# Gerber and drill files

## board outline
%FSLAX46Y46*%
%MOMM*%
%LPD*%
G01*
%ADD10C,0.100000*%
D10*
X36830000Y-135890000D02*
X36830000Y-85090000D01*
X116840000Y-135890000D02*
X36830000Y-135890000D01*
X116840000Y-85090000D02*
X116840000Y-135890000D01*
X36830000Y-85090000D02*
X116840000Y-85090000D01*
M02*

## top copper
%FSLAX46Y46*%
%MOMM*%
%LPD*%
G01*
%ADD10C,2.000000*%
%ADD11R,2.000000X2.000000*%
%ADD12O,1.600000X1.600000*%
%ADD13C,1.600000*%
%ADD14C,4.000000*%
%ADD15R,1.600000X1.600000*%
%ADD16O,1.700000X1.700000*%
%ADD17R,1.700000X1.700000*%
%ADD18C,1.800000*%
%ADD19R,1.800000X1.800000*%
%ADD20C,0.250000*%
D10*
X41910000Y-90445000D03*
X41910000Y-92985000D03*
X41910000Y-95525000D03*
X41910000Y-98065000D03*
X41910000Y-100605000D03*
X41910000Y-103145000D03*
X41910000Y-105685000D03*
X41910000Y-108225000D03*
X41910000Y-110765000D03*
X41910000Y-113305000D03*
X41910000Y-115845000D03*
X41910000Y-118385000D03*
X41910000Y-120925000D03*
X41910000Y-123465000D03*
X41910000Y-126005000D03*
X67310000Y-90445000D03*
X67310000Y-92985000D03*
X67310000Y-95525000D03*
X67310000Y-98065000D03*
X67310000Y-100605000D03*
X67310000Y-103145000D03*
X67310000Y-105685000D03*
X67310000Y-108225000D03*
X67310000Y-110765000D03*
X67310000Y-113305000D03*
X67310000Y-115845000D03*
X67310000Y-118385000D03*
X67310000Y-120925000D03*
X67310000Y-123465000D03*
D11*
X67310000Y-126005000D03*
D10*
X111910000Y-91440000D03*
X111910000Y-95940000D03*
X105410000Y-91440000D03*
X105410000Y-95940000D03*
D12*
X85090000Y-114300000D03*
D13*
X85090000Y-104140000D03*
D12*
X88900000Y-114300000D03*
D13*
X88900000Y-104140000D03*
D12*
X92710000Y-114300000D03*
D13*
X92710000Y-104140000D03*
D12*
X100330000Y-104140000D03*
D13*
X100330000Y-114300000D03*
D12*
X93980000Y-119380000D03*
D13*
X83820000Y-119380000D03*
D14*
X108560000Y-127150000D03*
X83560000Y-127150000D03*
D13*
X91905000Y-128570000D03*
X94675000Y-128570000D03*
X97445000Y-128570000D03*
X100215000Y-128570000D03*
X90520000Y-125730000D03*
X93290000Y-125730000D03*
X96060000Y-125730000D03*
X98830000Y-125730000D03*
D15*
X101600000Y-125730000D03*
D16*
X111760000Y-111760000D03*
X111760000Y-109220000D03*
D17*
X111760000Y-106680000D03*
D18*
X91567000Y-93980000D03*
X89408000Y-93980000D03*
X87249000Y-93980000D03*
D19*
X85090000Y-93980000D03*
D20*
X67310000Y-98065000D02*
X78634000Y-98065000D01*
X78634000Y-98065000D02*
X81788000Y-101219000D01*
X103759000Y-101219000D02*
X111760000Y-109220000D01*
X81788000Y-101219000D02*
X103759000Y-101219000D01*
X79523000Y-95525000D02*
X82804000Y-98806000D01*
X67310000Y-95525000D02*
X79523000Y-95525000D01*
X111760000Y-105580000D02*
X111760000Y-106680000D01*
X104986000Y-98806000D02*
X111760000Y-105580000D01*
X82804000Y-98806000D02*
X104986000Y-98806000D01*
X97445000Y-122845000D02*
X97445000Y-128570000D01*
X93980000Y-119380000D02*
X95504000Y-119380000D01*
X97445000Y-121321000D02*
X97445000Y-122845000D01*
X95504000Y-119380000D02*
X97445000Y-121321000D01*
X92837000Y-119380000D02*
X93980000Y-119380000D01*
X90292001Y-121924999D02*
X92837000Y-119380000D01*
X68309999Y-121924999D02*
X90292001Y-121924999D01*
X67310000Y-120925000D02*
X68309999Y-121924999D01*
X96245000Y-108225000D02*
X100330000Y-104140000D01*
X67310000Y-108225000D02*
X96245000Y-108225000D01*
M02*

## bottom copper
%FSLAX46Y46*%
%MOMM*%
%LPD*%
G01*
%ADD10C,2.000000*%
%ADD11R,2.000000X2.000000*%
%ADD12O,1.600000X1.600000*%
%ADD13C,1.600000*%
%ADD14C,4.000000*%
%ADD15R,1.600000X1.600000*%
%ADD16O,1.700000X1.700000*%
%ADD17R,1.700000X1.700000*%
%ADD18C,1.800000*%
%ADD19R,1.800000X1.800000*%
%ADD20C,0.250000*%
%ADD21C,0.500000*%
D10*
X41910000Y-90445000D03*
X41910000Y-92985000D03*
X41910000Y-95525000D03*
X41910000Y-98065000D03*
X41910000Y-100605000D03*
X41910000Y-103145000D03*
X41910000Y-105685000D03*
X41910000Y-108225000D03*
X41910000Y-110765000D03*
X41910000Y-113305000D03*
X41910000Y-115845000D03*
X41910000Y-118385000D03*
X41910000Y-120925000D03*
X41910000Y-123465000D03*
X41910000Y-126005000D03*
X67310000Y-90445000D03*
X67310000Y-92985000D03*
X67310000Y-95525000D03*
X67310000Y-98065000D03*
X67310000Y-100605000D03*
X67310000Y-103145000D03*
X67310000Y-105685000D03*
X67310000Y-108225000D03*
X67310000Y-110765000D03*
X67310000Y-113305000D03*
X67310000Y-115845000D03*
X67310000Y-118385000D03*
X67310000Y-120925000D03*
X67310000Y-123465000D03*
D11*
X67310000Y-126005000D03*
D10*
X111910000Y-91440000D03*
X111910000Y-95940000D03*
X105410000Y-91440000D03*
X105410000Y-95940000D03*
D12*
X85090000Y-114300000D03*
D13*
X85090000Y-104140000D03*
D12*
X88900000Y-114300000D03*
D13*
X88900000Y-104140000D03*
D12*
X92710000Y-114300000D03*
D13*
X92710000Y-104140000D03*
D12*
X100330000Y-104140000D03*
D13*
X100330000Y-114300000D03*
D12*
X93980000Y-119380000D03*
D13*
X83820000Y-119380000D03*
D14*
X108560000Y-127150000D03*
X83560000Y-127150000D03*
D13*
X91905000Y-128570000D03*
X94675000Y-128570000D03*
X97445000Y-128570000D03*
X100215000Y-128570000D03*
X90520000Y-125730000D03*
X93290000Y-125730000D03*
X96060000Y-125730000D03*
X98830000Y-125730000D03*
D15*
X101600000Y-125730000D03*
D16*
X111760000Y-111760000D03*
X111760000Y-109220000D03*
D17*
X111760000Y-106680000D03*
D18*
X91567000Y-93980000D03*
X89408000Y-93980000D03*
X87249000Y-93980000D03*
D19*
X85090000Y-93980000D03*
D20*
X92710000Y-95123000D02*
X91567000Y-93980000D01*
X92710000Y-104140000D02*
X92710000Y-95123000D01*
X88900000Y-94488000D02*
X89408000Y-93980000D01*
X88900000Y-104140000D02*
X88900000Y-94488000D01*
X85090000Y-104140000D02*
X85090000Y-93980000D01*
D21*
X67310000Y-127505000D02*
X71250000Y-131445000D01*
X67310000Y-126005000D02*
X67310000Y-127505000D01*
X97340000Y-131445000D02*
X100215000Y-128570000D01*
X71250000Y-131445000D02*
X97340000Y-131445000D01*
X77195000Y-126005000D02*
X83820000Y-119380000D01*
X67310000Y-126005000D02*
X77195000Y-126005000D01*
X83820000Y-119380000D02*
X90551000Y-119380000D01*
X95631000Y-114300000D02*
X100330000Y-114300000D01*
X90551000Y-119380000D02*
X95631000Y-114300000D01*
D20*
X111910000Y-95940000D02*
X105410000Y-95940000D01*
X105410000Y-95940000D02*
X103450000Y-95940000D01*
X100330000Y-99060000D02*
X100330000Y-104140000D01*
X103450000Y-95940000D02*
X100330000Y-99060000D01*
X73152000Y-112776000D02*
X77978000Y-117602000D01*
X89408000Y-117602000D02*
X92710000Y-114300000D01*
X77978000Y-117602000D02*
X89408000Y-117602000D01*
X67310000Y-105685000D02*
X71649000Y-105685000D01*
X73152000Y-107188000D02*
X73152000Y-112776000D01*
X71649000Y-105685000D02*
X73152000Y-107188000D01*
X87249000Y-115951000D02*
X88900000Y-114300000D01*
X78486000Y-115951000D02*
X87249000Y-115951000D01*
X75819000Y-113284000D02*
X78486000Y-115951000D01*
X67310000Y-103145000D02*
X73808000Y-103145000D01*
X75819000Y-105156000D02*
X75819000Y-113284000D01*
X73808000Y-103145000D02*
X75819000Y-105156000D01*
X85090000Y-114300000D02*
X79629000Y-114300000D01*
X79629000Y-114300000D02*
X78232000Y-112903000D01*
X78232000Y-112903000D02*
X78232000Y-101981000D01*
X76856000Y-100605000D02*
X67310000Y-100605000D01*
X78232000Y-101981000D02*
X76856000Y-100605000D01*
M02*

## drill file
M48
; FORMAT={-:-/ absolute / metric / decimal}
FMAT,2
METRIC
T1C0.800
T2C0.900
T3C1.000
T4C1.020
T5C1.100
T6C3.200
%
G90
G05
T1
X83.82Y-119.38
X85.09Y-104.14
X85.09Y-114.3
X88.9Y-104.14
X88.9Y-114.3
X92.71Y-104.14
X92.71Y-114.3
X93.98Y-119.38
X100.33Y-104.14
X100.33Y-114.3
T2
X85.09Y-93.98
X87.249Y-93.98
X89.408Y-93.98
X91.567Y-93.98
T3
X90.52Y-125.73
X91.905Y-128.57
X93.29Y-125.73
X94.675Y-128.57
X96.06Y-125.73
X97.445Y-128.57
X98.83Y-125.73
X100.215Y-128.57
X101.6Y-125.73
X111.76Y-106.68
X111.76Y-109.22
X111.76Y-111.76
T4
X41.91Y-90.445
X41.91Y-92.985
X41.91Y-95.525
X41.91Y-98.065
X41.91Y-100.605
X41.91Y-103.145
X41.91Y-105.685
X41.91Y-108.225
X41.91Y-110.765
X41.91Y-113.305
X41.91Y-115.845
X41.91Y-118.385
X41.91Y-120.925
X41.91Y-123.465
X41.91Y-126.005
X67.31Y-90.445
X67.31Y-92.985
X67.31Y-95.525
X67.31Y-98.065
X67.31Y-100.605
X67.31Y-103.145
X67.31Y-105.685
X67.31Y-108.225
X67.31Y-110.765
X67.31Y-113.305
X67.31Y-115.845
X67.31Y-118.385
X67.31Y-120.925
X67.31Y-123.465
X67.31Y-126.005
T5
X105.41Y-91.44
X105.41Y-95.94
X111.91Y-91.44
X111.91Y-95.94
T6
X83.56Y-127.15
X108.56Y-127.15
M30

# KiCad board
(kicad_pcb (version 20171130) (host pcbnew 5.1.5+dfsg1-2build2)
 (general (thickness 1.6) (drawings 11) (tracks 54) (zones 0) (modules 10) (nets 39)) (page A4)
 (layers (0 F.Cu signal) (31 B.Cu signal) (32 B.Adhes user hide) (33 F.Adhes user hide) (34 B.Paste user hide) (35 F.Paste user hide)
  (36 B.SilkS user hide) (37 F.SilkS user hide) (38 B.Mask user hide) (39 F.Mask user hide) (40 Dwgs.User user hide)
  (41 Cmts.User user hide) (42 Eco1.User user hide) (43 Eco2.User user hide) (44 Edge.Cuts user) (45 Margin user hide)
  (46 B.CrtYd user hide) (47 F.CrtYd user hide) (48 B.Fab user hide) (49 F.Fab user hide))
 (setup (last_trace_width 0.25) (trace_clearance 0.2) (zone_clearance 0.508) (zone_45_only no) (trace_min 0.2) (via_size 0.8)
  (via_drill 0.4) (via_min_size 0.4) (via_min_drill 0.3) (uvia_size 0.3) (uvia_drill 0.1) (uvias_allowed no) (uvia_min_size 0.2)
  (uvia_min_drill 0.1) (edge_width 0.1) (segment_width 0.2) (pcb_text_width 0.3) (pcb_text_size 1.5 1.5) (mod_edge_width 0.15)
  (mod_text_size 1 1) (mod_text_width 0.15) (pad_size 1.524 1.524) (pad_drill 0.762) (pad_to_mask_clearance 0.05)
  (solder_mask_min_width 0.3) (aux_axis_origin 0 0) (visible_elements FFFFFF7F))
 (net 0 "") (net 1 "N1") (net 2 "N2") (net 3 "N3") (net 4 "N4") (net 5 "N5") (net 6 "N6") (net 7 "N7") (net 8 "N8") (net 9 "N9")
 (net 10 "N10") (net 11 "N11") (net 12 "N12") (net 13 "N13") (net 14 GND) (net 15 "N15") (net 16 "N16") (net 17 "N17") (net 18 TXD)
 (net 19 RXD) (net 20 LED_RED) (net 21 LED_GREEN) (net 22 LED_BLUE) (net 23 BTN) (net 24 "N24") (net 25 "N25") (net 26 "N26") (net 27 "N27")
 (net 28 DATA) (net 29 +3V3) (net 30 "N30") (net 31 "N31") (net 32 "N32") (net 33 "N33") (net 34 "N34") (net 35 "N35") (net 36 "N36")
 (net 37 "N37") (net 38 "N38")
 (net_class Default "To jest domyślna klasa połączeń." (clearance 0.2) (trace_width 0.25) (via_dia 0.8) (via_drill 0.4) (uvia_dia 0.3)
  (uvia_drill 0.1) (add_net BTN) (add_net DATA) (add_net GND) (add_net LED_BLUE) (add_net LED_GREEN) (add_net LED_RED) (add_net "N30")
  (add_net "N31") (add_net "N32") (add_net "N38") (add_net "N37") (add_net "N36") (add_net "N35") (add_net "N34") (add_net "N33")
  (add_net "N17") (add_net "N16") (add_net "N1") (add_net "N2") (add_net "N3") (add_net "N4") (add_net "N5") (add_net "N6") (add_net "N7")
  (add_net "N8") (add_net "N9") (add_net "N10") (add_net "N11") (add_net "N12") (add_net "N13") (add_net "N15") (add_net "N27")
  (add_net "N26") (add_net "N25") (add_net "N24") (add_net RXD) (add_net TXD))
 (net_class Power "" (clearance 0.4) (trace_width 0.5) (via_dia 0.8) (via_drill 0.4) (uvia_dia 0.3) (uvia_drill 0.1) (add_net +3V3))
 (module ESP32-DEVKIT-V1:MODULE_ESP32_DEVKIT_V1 (layer F.Cu) (at 54.61 110.49 180)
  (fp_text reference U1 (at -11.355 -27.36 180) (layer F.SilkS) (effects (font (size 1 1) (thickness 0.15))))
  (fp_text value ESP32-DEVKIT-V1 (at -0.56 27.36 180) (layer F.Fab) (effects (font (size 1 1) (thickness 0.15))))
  (pad 16 thru_hole circle (at 12.7 20.045 180) (size 2 2) (drill 1.02) (layers *.Cu *.Mask) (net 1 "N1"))
  (pad 17 thru_hole circle (at 12.7 17.505 180) (size 2 2) (drill 1.02) (layers *.Cu *.Mask) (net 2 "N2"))
  (pad 18 thru_hole circle (at 12.7 14.965 180) (size 2 2) (drill 1.02) (layers *.Cu *.Mask) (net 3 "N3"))
  (pad 19 thru_hole circle (at 12.7 12.425 180) (size 2 2) (drill 1.02) (layers *.Cu *.Mask) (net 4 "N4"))
  (pad 20 thru_hole circle (at 12.7 9.885 180) (size 2 2) (drill 1.02) (layers *.Cu *.Mask) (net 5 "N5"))
  (pad 21 thru_hole circle (at 12.7 7.345 180) (size 2 2) (drill 1.02) (layers *.Cu *.Mask) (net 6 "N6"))
  (pad 22 thru_hole circle (at 12.7 4.805 180) (size 2 2) (drill 1.02) (layers *.Cu *.Mask) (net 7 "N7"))
  (pad 23 thru_hole circle (at 12.7 2.265 180) (size 2 2) (drill 1.02) (layers *.Cu *.Mask) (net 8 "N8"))
  (pad 24 thru_hole circle (at 12.7 -0.275 180) (size 2 2) (drill 1.02) (layers *.Cu *.Mask) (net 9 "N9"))
  (pad 25 thru_hole circle (at 12.7 -2.815 180) (size 2 2) (drill 1.02) (layers *.Cu *.Mask) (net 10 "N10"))
  (pad 26 thru_hole circle (at 12.7 -5.355 180) (size 2 2) (drill 1.02) (layers *.Cu *.Mask) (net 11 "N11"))
  (pad 27 thru_hole circle (at 12.7 -7.895 180) (size 2 2) (drill 1.02) (layers *.Cu *.Mask) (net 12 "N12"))
  (pad 28 thru_hole circle (at 12.7 -10.435 180) (size 2 2) (drill 1.02) (layers *.Cu *.Mask) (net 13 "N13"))
  (pad 29 thru_hole circle (at 12.7 -12.975 180) (size 2 2) (drill 1.02) (layers *.Cu *.Mask) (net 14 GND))
  (pad 30 thru_hole circle (at 12.7 -15.515 180) (size 2 2) (drill 1.02) (layers *.Cu *.Mask) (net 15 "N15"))
  (pad 15 thru_hole circle (at -12.7 20.045 180) (size 2 2) (drill 1.02) (layers *.Cu *.Mask) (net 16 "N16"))
  (pad 14 thru_hole circle (at -12.7 17.505 180) (size 2 2) (drill 1.02) (layers *.Cu *.Mask) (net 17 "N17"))
  (pad 13 thru_hole circle (at -12.7 14.965 180) (size 2 2) (drill 1.02) (layers *.Cu *.Mask) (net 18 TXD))
  (pad 12 thru_hole circle (at -12.7 12.425 180) (size 2 2) (drill 1.02) (layers *.Cu *.Mask) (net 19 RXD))
  (pad 11 thru_hole circle (at -12.7 9.885 180) (size 2 2) (drill 1.02) (layers *.Cu *.Mask) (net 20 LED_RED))
  (pad 10 thru_hole circle (at -12.7 7.345 180) (size 2 2) (drill 1.02) (layers *.Cu *.Mask) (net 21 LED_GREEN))
  (pad 9 thru_hole circle (at -12.7 4.805 180) (size 2 2) (drill 1.02) (layers *.Cu *.Mask) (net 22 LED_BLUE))
  (pad 8 thru_hole circle (at -12.7 2.265 180) (size 2 2) (drill 1.02) (layers *.Cu *.Mask) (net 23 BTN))
  (pad 7 thru_hole circle (at -12.7 -0.275 180) (size 2 2) (drill 1.02) (layers *.Cu *.Mask) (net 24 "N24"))
  (pad 6 thru_hole circle (at -12.7 -2.815 180) (size 2 2) (drill 1.02) (layers *.Cu *.Mask) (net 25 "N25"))
  (pad 5 thru_hole circle (at -12.7 -5.355 180) (size 2 2) (drill 1.02) (layers *.Cu *.Mask) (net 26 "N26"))
  (pad 4 thru_hole circle (at -12.7 -7.895 180) (size 2 2) (drill 1.02) (layers *.Cu *.Mask) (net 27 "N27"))
  (pad 3 thru_hole circle (at -12.7 -10.435 180) (size 2 2) (drill 1.02) (layers *.Cu *.Mask) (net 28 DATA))
  (pad 2 thru_hole circle (at -12.7 -12.975 180) (size 2 2) (drill 1.02) (layers *.Cu *.Mask) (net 14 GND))
  (pad 1 thru_hole rect (at -12.7 -15.515 180) (size 2 2) (drill 1.02) (layers *.Cu *.Mask) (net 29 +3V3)))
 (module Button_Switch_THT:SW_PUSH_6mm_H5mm (layer F.Cu) (at 105.41 91.44)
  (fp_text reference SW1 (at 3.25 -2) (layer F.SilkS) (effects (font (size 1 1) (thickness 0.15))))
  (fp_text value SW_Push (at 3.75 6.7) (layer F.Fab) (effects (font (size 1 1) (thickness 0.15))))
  (pad 1 thru_hole circle (at 6.5 0 90) (size 2 2) (drill 1.1) (layers *.Cu *.Mask) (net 14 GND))
  (pad 2 thru_hole circle (at 6.5 4.5 90) (size 2 2) (drill 1.1) (layers *.Cu *.Mask) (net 23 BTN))
  (pad 1 thru_hole circle (at 0 0 90) (size 2 2) (drill 1.1) (layers *.Cu *.Mask) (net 14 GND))
  (pad 2 thru_hole circle (at 0 4.5 90) (size 2 2) (drill 1.1) (layers *.Cu *.Mask) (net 23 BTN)))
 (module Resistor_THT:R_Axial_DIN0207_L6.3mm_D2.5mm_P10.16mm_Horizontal (layer F.Cu) (at 85.09 104.14 270)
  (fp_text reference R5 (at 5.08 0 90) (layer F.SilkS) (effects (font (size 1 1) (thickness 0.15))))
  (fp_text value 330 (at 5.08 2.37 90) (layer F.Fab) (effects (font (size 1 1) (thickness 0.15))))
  (pad 2 thru_hole oval (at 10.16 0 270) (size 1.6 1.6) (drill 0.8) (layers *.Cu *.Mask) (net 20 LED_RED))
  (pad 1 thru_hole circle (at 0 0 270) (size 1.6 1.6) (drill 0.8) (layers *.Cu *.Mask) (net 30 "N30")))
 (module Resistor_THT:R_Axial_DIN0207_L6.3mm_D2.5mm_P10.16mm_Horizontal (layer F.Cu) (at 88.9 104.14 270)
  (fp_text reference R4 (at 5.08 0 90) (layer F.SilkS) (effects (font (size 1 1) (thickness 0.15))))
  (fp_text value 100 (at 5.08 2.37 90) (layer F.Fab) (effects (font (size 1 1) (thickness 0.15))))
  (pad 2 thru_hole oval (at 10.16 0 270) (size 1.6 1.6) (drill 0.8) (layers *.Cu *.Mask) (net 21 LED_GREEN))
  (pad 1 thru_hole circle (at 0 0 270) (size 1.6 1.6) (drill 0.8) (layers *.Cu *.Mask) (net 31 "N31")))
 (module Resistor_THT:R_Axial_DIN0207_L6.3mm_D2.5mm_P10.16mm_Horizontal (layer F.Cu) (at 92.71 104.14 270)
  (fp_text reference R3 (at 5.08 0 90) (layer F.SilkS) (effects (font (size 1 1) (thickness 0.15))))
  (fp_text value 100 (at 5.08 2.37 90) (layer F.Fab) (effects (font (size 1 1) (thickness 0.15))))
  (pad 2 thru_hole oval (at 10.16 0 270) (size 1.6 1.6) (drill 0.8) (layers *.Cu *.Mask) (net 22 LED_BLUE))
  (pad 1 thru_hole circle (at 0 0 270) (size 1.6 1.6) (drill 0.8) (layers *.Cu *.Mask) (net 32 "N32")))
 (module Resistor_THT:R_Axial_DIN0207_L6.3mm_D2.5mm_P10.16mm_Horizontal (layer F.Cu) (at 100.33 114.3 90)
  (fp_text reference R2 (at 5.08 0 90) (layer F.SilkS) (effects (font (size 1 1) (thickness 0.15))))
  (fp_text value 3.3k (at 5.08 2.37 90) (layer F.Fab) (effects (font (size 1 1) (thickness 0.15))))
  (pad 2 thru_hole oval (at 10.16 0 90) (size 1.6 1.6) (drill 0.8) (layers *.Cu *.Mask) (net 23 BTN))
  (pad 1 thru_hole circle (at 0 0 90) (size 1.6 1.6) (drill 0.8) (layers *.Cu *.Mask) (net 29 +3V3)))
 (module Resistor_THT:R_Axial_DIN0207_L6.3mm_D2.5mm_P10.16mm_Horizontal (layer F.Cu) (at 83.82 119.38)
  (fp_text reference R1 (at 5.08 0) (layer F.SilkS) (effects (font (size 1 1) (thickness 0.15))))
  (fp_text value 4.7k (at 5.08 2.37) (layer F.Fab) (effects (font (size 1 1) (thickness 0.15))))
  (pad 2 thru_hole oval (at 10.16 0) (size 1.6 1.6) (drill 0.8) (layers *.Cu *.Mask) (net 28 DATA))
  (pad 1 thru_hole circle (at 0 0) (size 1.6 1.6) (drill 0.8) (layers *.Cu *.Mask) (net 29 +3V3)))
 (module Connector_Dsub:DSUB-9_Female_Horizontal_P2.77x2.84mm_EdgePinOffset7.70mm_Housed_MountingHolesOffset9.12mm (layer F.Cu)
  (at 101.6 125.73)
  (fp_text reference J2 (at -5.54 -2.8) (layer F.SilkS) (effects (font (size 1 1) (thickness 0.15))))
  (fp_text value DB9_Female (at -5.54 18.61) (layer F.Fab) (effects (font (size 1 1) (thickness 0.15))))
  (pad 0 thru_hole circle (at 6.96 1.42) (size 4 4) (drill 3.2) (layers *.Cu *.Mask))
  (pad 0 thru_hole circle (at -18.04 1.42) (size 4 4) (drill 3.2) (layers *.Cu *.Mask))
  (pad 9 thru_hole circle (at -9.695 2.84) (size 1.6 1.6) (drill 1) (layers *.Cu *.Mask) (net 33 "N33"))
  (pad 8 thru_hole circle (at -6.925 2.84) (size 1.6 1.6) (drill 1) (layers *.Cu *.Mask) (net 14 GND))
  (pad 7 thru_hole circle (at -4.155 2.84) (size 1.6 1.6) (drill 1) (layers *.Cu *.Mask) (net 28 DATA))
  (pad 6 thru_hole circle (at -1.385 2.84) (size 1.6 1.6) (drill 1) (layers *.Cu *.Mask) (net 29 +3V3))
  (pad 5 thru_hole circle (at -11.08 0) (size 1.6 1.6) (drill 1) (layers *.Cu *.Mask) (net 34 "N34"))
  (pad 4 thru_hole circle (at -8.31 0) (size 1.6 1.6) (drill 1) (layers *.Cu *.Mask) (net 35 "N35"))
  (pad 3 thru_hole circle (at -5.54 0) (size 1.6 1.6) (drill 1) (layers *.Cu *.Mask) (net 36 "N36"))
  (pad 2 thru_hole circle (at -2.77 0) (size 1.6 1.6) (drill 1) (layers *.Cu *.Mask) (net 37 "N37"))
  (pad 1 thru_hole rect (at 0 0) (size 1.6 1.6) (drill 1) (layers *.Cu *.Mask) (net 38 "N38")))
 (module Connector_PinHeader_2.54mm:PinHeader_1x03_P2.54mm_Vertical (layer F.Cu) (at 111.76 106.68)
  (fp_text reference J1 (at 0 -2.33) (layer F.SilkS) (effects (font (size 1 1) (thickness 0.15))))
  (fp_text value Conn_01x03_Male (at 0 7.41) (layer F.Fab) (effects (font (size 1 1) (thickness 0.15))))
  (pad 3 thru_hole oval (at 0 5.08) (size 1.7 1.7) (drill 1) (layers *.Cu *.Mask) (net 14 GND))
  (pad 2 thru_hole oval (at 0 2.54) (size 1.7 1.7) (drill 1) (layers *.Cu *.Mask) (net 19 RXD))
  (pad 1 thru_hole rect (at 0 0) (size 1.7 1.7) (drill 1) (layers *.Cu *.Mask) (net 18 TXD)))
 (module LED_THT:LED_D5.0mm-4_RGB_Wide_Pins (layer F.Cu) (at 85.09 93.98)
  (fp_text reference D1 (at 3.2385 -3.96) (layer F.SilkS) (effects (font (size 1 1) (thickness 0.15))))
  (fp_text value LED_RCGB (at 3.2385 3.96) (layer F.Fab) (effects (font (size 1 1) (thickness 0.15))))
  (pad 4 thru_hole circle (at 6.477 0) (size 1.8 1.8) (drill 0.9) (layers *.Cu *.Mask) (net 32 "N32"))
  (pad 3 thru_hole circle (at 4.318 0) (size 1.8 1.8) (drill 0.9) (layers *.Cu *.Mask) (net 31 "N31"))
  (pad 2 thru_hole circle (at 2.159 0) (size 1.8 1.8) (drill 0.9) (layers *.Cu *.Mask) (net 14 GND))
  (pad 1 thru_hole rect (at 0 0) (size 1.8 1.8) (drill 0.9) (layers *.Cu *.Mask) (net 30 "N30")))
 (gr_line (start 36.83 135.89) (end 36.83 85.09) (layer Edge.Cuts) (width 0.1))
 (gr_line (start 116.84 135.89) (end 36.83 135.89) (layer Edge.Cuts) (width 0.1))
 (gr_line (start 116.84 85.09) (end 116.84 135.89) (layer Edge.Cuts) (width 0.1))
 (gr_line (start 36.83 85.09) (end 116.84 85.09) (layer Edge.Cuts) (width 0.1))
 (segment (start 92.71 95.123) (end 91.567 93.98) (width 0.25) (layer B.Cu) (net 32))
 (segment (start 92.71 104.14) (end 92.71 95.123) (width 0.25) (layer B.Cu) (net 32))
 (segment (start 88.9 94.488) (end 89.408 93.98) (width 0.25) (layer B.Cu) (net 31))
 (segment (start 88.9 104.14) (end 88.9 94.488) (width 0.25) (layer B.Cu) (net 31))
 (segment (start 85.09 104.14) (end 85.09 93.98) (width 0.25) (layer B.Cu) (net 30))
 (segment (start 67.31 98.065) (end 78.634 98.065) (width 0.25) (layer F.Cu) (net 19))
 (segment (start 78.634 98.065) (end 81.788 101.219) (width 0.25) (layer F.Cu) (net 19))
 (segment (start 103.759 101.219) (end 111.76 109.22) (width 0.25) (layer F.Cu) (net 19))
 (segment (start 81.788 101.219) (end 103.759 101.219) (width 0.25) (layer F.Cu) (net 19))
 (segment (start 79.523 95.525) (end 82.804 98.806) (width 0.25) (layer F.Cu) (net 18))
 (segment (start 67.31 95.525) (end 79.523 95.525) (width 0.25) (layer F.Cu) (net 18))
 (segment (start 111.76 105.58) (end 111.76 106.68) (width 0.25) (layer F.Cu) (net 18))
 (segment (start 104.986 98.806) (end 111.76 105.58) (width 0.25) (layer F.Cu) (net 18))
 (segment (start 82.804 98.806) (end 104.986 98.806) (width 0.25) (layer F.Cu) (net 18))
 (segment (start 97.445 122.845) (end 97.445 128.57) (width 0.25) (layer F.Cu) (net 28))
 (segment (start 93.98 119.38) (end 95.504 119.38) (width 0.25) (layer F.Cu) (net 28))
 (segment (start 97.445 121.321) (end 97.445 122.845) (width 0.25) (layer F.Cu) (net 28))
 (segment (start 95.504 119.38) (end 97.445 121.321) (width 0.25) (layer F.Cu) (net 28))
 (segment (start 92.837 119.38) (end 93.98 119.38) (width 0.25) (layer F.Cu) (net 28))
 (segment (start 90.292001 121.924999) (end 92.837 119.38) (width 0.25) (layer F.Cu) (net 28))
 (segment (start 68.309999 121.924999) (end 90.292001 121.924999) (width 0.25) (layer F.Cu) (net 28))
 (segment (start 67.31 120.925) (end 68.309999 121.924999) (width 0.25) (layer F.Cu) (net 28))
 (segment (start 67.31 127.505) (end 71.25 131.445) (width 0.5) (layer B.Cu) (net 29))
 (segment (start 67.31 126.005) (end 67.31 127.505) (width 0.5) (layer B.Cu) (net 29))
 (segment (start 97.34 131.445) (end 100.215 128.57) (width 0.5) (layer B.Cu) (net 29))
 (segment (start 71.25 131.445) (end 97.34 131.445) (width 0.5) (layer B.Cu) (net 29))
 (segment (start 77.195 126.005) (end 83.82 119.38) (width 0.5) (layer B.Cu) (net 29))
 (segment (start 67.31 126.005) (end 77.195 126.005) (width 0.5) (layer B.Cu) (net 29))
 (segment (start 83.82 119.38) (end 90.551 119.38) (width 0.5) (layer B.Cu) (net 29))
 (segment (start 95.631 114.3) (end 100.33 114.3) (width 0.5) (layer B.Cu) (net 29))
 (segment (start 90.551 119.38) (end 95.631 114.3) (width 0.5) (layer B.Cu) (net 29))
 (segment (start 111.91 95.94) (end 105.41 95.94) (width 0.25) (layer B.Cu) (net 23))
 (segment (start 105.41 95.94) (end 103.45 95.94) (width 0.25) (layer B.Cu) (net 23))
 (segment (start 100.33 99.06) (end 100.33 104.14) (width 0.25) (layer B.Cu) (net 23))
 (segment (start 103.45 95.94) (end 100.33 99.06) (width 0.25) (layer B.Cu) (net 23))
 (segment (start 96.245 108.225) (end 100.33 104.14) (width 0.25) (layer F.Cu) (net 23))
 (segment (start 67.31 108.225) (end 96.245 108.225) (width 0.25) (layer F.Cu) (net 23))
 (segment (start 73.152 112.776) (end 77.978 117.602) (width 0.25) (layer B.Cu) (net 22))
 (segment (start 89.408 117.602) (end 92.71 114.3) (width 0.25) (layer B.Cu) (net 22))
 (segment (start 77.978 117.602) (end 89.408 117.602) (width 0.25) (layer B.Cu) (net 22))
 (segment (start 67.31 105.685) (end 71.649 105.685) (width 0.25) (layer B.Cu) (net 22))
 (segment (start 73.152 107.188) (end 73.152 112.776) (width 0.25) (layer B.Cu) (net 22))
 (segment (start 71.649 105.685) (end 73.152 107.188) (width 0.25) (layer B.Cu) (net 22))
 (segment (start 87.249 115.951) (end 88.9 114.3) (width 0.25) (layer B.Cu) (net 21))
 (segment (start 78.486 115.951) (end 87.249 115.951) (width 0.25) (layer B.Cu) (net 21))
 (segment (start 75.819 113.284) (end 78.486 115.951) (width 0.25) (layer B.Cu) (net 21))
 (segment (start 67.31 103.145) (end 73.808 103.145) (width 0.25) (layer B.Cu) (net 21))
 (segment (start 75.819 105.156) (end 75.819 113.284) (width 0.25) (layer B.Cu) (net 21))
 (segment (start 73.808 103.145) (end 75.819 105.156) (width 0.25) (layer B.Cu) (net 21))
 (segment (start 85.09 114.3) (end 79.629 114.3) (width 0.25) (layer B.Cu) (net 20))
 (segment (start 79.629 114.3) (end 78.232 112.903) (width 0.25) (layer B.Cu) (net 20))
 (segment (start 78.232 112.903) (end 78.232 101.981) (width 0.25) (layer B.Cu) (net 20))
 (segment (start 76.856 100.605) (end 67.31 100.605) (width 0.25) (layer B.Cu) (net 20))
 (segment (start 78.232 101.981) (end 76.856 100.605) (width 0.25) (layer B.Cu) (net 20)))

